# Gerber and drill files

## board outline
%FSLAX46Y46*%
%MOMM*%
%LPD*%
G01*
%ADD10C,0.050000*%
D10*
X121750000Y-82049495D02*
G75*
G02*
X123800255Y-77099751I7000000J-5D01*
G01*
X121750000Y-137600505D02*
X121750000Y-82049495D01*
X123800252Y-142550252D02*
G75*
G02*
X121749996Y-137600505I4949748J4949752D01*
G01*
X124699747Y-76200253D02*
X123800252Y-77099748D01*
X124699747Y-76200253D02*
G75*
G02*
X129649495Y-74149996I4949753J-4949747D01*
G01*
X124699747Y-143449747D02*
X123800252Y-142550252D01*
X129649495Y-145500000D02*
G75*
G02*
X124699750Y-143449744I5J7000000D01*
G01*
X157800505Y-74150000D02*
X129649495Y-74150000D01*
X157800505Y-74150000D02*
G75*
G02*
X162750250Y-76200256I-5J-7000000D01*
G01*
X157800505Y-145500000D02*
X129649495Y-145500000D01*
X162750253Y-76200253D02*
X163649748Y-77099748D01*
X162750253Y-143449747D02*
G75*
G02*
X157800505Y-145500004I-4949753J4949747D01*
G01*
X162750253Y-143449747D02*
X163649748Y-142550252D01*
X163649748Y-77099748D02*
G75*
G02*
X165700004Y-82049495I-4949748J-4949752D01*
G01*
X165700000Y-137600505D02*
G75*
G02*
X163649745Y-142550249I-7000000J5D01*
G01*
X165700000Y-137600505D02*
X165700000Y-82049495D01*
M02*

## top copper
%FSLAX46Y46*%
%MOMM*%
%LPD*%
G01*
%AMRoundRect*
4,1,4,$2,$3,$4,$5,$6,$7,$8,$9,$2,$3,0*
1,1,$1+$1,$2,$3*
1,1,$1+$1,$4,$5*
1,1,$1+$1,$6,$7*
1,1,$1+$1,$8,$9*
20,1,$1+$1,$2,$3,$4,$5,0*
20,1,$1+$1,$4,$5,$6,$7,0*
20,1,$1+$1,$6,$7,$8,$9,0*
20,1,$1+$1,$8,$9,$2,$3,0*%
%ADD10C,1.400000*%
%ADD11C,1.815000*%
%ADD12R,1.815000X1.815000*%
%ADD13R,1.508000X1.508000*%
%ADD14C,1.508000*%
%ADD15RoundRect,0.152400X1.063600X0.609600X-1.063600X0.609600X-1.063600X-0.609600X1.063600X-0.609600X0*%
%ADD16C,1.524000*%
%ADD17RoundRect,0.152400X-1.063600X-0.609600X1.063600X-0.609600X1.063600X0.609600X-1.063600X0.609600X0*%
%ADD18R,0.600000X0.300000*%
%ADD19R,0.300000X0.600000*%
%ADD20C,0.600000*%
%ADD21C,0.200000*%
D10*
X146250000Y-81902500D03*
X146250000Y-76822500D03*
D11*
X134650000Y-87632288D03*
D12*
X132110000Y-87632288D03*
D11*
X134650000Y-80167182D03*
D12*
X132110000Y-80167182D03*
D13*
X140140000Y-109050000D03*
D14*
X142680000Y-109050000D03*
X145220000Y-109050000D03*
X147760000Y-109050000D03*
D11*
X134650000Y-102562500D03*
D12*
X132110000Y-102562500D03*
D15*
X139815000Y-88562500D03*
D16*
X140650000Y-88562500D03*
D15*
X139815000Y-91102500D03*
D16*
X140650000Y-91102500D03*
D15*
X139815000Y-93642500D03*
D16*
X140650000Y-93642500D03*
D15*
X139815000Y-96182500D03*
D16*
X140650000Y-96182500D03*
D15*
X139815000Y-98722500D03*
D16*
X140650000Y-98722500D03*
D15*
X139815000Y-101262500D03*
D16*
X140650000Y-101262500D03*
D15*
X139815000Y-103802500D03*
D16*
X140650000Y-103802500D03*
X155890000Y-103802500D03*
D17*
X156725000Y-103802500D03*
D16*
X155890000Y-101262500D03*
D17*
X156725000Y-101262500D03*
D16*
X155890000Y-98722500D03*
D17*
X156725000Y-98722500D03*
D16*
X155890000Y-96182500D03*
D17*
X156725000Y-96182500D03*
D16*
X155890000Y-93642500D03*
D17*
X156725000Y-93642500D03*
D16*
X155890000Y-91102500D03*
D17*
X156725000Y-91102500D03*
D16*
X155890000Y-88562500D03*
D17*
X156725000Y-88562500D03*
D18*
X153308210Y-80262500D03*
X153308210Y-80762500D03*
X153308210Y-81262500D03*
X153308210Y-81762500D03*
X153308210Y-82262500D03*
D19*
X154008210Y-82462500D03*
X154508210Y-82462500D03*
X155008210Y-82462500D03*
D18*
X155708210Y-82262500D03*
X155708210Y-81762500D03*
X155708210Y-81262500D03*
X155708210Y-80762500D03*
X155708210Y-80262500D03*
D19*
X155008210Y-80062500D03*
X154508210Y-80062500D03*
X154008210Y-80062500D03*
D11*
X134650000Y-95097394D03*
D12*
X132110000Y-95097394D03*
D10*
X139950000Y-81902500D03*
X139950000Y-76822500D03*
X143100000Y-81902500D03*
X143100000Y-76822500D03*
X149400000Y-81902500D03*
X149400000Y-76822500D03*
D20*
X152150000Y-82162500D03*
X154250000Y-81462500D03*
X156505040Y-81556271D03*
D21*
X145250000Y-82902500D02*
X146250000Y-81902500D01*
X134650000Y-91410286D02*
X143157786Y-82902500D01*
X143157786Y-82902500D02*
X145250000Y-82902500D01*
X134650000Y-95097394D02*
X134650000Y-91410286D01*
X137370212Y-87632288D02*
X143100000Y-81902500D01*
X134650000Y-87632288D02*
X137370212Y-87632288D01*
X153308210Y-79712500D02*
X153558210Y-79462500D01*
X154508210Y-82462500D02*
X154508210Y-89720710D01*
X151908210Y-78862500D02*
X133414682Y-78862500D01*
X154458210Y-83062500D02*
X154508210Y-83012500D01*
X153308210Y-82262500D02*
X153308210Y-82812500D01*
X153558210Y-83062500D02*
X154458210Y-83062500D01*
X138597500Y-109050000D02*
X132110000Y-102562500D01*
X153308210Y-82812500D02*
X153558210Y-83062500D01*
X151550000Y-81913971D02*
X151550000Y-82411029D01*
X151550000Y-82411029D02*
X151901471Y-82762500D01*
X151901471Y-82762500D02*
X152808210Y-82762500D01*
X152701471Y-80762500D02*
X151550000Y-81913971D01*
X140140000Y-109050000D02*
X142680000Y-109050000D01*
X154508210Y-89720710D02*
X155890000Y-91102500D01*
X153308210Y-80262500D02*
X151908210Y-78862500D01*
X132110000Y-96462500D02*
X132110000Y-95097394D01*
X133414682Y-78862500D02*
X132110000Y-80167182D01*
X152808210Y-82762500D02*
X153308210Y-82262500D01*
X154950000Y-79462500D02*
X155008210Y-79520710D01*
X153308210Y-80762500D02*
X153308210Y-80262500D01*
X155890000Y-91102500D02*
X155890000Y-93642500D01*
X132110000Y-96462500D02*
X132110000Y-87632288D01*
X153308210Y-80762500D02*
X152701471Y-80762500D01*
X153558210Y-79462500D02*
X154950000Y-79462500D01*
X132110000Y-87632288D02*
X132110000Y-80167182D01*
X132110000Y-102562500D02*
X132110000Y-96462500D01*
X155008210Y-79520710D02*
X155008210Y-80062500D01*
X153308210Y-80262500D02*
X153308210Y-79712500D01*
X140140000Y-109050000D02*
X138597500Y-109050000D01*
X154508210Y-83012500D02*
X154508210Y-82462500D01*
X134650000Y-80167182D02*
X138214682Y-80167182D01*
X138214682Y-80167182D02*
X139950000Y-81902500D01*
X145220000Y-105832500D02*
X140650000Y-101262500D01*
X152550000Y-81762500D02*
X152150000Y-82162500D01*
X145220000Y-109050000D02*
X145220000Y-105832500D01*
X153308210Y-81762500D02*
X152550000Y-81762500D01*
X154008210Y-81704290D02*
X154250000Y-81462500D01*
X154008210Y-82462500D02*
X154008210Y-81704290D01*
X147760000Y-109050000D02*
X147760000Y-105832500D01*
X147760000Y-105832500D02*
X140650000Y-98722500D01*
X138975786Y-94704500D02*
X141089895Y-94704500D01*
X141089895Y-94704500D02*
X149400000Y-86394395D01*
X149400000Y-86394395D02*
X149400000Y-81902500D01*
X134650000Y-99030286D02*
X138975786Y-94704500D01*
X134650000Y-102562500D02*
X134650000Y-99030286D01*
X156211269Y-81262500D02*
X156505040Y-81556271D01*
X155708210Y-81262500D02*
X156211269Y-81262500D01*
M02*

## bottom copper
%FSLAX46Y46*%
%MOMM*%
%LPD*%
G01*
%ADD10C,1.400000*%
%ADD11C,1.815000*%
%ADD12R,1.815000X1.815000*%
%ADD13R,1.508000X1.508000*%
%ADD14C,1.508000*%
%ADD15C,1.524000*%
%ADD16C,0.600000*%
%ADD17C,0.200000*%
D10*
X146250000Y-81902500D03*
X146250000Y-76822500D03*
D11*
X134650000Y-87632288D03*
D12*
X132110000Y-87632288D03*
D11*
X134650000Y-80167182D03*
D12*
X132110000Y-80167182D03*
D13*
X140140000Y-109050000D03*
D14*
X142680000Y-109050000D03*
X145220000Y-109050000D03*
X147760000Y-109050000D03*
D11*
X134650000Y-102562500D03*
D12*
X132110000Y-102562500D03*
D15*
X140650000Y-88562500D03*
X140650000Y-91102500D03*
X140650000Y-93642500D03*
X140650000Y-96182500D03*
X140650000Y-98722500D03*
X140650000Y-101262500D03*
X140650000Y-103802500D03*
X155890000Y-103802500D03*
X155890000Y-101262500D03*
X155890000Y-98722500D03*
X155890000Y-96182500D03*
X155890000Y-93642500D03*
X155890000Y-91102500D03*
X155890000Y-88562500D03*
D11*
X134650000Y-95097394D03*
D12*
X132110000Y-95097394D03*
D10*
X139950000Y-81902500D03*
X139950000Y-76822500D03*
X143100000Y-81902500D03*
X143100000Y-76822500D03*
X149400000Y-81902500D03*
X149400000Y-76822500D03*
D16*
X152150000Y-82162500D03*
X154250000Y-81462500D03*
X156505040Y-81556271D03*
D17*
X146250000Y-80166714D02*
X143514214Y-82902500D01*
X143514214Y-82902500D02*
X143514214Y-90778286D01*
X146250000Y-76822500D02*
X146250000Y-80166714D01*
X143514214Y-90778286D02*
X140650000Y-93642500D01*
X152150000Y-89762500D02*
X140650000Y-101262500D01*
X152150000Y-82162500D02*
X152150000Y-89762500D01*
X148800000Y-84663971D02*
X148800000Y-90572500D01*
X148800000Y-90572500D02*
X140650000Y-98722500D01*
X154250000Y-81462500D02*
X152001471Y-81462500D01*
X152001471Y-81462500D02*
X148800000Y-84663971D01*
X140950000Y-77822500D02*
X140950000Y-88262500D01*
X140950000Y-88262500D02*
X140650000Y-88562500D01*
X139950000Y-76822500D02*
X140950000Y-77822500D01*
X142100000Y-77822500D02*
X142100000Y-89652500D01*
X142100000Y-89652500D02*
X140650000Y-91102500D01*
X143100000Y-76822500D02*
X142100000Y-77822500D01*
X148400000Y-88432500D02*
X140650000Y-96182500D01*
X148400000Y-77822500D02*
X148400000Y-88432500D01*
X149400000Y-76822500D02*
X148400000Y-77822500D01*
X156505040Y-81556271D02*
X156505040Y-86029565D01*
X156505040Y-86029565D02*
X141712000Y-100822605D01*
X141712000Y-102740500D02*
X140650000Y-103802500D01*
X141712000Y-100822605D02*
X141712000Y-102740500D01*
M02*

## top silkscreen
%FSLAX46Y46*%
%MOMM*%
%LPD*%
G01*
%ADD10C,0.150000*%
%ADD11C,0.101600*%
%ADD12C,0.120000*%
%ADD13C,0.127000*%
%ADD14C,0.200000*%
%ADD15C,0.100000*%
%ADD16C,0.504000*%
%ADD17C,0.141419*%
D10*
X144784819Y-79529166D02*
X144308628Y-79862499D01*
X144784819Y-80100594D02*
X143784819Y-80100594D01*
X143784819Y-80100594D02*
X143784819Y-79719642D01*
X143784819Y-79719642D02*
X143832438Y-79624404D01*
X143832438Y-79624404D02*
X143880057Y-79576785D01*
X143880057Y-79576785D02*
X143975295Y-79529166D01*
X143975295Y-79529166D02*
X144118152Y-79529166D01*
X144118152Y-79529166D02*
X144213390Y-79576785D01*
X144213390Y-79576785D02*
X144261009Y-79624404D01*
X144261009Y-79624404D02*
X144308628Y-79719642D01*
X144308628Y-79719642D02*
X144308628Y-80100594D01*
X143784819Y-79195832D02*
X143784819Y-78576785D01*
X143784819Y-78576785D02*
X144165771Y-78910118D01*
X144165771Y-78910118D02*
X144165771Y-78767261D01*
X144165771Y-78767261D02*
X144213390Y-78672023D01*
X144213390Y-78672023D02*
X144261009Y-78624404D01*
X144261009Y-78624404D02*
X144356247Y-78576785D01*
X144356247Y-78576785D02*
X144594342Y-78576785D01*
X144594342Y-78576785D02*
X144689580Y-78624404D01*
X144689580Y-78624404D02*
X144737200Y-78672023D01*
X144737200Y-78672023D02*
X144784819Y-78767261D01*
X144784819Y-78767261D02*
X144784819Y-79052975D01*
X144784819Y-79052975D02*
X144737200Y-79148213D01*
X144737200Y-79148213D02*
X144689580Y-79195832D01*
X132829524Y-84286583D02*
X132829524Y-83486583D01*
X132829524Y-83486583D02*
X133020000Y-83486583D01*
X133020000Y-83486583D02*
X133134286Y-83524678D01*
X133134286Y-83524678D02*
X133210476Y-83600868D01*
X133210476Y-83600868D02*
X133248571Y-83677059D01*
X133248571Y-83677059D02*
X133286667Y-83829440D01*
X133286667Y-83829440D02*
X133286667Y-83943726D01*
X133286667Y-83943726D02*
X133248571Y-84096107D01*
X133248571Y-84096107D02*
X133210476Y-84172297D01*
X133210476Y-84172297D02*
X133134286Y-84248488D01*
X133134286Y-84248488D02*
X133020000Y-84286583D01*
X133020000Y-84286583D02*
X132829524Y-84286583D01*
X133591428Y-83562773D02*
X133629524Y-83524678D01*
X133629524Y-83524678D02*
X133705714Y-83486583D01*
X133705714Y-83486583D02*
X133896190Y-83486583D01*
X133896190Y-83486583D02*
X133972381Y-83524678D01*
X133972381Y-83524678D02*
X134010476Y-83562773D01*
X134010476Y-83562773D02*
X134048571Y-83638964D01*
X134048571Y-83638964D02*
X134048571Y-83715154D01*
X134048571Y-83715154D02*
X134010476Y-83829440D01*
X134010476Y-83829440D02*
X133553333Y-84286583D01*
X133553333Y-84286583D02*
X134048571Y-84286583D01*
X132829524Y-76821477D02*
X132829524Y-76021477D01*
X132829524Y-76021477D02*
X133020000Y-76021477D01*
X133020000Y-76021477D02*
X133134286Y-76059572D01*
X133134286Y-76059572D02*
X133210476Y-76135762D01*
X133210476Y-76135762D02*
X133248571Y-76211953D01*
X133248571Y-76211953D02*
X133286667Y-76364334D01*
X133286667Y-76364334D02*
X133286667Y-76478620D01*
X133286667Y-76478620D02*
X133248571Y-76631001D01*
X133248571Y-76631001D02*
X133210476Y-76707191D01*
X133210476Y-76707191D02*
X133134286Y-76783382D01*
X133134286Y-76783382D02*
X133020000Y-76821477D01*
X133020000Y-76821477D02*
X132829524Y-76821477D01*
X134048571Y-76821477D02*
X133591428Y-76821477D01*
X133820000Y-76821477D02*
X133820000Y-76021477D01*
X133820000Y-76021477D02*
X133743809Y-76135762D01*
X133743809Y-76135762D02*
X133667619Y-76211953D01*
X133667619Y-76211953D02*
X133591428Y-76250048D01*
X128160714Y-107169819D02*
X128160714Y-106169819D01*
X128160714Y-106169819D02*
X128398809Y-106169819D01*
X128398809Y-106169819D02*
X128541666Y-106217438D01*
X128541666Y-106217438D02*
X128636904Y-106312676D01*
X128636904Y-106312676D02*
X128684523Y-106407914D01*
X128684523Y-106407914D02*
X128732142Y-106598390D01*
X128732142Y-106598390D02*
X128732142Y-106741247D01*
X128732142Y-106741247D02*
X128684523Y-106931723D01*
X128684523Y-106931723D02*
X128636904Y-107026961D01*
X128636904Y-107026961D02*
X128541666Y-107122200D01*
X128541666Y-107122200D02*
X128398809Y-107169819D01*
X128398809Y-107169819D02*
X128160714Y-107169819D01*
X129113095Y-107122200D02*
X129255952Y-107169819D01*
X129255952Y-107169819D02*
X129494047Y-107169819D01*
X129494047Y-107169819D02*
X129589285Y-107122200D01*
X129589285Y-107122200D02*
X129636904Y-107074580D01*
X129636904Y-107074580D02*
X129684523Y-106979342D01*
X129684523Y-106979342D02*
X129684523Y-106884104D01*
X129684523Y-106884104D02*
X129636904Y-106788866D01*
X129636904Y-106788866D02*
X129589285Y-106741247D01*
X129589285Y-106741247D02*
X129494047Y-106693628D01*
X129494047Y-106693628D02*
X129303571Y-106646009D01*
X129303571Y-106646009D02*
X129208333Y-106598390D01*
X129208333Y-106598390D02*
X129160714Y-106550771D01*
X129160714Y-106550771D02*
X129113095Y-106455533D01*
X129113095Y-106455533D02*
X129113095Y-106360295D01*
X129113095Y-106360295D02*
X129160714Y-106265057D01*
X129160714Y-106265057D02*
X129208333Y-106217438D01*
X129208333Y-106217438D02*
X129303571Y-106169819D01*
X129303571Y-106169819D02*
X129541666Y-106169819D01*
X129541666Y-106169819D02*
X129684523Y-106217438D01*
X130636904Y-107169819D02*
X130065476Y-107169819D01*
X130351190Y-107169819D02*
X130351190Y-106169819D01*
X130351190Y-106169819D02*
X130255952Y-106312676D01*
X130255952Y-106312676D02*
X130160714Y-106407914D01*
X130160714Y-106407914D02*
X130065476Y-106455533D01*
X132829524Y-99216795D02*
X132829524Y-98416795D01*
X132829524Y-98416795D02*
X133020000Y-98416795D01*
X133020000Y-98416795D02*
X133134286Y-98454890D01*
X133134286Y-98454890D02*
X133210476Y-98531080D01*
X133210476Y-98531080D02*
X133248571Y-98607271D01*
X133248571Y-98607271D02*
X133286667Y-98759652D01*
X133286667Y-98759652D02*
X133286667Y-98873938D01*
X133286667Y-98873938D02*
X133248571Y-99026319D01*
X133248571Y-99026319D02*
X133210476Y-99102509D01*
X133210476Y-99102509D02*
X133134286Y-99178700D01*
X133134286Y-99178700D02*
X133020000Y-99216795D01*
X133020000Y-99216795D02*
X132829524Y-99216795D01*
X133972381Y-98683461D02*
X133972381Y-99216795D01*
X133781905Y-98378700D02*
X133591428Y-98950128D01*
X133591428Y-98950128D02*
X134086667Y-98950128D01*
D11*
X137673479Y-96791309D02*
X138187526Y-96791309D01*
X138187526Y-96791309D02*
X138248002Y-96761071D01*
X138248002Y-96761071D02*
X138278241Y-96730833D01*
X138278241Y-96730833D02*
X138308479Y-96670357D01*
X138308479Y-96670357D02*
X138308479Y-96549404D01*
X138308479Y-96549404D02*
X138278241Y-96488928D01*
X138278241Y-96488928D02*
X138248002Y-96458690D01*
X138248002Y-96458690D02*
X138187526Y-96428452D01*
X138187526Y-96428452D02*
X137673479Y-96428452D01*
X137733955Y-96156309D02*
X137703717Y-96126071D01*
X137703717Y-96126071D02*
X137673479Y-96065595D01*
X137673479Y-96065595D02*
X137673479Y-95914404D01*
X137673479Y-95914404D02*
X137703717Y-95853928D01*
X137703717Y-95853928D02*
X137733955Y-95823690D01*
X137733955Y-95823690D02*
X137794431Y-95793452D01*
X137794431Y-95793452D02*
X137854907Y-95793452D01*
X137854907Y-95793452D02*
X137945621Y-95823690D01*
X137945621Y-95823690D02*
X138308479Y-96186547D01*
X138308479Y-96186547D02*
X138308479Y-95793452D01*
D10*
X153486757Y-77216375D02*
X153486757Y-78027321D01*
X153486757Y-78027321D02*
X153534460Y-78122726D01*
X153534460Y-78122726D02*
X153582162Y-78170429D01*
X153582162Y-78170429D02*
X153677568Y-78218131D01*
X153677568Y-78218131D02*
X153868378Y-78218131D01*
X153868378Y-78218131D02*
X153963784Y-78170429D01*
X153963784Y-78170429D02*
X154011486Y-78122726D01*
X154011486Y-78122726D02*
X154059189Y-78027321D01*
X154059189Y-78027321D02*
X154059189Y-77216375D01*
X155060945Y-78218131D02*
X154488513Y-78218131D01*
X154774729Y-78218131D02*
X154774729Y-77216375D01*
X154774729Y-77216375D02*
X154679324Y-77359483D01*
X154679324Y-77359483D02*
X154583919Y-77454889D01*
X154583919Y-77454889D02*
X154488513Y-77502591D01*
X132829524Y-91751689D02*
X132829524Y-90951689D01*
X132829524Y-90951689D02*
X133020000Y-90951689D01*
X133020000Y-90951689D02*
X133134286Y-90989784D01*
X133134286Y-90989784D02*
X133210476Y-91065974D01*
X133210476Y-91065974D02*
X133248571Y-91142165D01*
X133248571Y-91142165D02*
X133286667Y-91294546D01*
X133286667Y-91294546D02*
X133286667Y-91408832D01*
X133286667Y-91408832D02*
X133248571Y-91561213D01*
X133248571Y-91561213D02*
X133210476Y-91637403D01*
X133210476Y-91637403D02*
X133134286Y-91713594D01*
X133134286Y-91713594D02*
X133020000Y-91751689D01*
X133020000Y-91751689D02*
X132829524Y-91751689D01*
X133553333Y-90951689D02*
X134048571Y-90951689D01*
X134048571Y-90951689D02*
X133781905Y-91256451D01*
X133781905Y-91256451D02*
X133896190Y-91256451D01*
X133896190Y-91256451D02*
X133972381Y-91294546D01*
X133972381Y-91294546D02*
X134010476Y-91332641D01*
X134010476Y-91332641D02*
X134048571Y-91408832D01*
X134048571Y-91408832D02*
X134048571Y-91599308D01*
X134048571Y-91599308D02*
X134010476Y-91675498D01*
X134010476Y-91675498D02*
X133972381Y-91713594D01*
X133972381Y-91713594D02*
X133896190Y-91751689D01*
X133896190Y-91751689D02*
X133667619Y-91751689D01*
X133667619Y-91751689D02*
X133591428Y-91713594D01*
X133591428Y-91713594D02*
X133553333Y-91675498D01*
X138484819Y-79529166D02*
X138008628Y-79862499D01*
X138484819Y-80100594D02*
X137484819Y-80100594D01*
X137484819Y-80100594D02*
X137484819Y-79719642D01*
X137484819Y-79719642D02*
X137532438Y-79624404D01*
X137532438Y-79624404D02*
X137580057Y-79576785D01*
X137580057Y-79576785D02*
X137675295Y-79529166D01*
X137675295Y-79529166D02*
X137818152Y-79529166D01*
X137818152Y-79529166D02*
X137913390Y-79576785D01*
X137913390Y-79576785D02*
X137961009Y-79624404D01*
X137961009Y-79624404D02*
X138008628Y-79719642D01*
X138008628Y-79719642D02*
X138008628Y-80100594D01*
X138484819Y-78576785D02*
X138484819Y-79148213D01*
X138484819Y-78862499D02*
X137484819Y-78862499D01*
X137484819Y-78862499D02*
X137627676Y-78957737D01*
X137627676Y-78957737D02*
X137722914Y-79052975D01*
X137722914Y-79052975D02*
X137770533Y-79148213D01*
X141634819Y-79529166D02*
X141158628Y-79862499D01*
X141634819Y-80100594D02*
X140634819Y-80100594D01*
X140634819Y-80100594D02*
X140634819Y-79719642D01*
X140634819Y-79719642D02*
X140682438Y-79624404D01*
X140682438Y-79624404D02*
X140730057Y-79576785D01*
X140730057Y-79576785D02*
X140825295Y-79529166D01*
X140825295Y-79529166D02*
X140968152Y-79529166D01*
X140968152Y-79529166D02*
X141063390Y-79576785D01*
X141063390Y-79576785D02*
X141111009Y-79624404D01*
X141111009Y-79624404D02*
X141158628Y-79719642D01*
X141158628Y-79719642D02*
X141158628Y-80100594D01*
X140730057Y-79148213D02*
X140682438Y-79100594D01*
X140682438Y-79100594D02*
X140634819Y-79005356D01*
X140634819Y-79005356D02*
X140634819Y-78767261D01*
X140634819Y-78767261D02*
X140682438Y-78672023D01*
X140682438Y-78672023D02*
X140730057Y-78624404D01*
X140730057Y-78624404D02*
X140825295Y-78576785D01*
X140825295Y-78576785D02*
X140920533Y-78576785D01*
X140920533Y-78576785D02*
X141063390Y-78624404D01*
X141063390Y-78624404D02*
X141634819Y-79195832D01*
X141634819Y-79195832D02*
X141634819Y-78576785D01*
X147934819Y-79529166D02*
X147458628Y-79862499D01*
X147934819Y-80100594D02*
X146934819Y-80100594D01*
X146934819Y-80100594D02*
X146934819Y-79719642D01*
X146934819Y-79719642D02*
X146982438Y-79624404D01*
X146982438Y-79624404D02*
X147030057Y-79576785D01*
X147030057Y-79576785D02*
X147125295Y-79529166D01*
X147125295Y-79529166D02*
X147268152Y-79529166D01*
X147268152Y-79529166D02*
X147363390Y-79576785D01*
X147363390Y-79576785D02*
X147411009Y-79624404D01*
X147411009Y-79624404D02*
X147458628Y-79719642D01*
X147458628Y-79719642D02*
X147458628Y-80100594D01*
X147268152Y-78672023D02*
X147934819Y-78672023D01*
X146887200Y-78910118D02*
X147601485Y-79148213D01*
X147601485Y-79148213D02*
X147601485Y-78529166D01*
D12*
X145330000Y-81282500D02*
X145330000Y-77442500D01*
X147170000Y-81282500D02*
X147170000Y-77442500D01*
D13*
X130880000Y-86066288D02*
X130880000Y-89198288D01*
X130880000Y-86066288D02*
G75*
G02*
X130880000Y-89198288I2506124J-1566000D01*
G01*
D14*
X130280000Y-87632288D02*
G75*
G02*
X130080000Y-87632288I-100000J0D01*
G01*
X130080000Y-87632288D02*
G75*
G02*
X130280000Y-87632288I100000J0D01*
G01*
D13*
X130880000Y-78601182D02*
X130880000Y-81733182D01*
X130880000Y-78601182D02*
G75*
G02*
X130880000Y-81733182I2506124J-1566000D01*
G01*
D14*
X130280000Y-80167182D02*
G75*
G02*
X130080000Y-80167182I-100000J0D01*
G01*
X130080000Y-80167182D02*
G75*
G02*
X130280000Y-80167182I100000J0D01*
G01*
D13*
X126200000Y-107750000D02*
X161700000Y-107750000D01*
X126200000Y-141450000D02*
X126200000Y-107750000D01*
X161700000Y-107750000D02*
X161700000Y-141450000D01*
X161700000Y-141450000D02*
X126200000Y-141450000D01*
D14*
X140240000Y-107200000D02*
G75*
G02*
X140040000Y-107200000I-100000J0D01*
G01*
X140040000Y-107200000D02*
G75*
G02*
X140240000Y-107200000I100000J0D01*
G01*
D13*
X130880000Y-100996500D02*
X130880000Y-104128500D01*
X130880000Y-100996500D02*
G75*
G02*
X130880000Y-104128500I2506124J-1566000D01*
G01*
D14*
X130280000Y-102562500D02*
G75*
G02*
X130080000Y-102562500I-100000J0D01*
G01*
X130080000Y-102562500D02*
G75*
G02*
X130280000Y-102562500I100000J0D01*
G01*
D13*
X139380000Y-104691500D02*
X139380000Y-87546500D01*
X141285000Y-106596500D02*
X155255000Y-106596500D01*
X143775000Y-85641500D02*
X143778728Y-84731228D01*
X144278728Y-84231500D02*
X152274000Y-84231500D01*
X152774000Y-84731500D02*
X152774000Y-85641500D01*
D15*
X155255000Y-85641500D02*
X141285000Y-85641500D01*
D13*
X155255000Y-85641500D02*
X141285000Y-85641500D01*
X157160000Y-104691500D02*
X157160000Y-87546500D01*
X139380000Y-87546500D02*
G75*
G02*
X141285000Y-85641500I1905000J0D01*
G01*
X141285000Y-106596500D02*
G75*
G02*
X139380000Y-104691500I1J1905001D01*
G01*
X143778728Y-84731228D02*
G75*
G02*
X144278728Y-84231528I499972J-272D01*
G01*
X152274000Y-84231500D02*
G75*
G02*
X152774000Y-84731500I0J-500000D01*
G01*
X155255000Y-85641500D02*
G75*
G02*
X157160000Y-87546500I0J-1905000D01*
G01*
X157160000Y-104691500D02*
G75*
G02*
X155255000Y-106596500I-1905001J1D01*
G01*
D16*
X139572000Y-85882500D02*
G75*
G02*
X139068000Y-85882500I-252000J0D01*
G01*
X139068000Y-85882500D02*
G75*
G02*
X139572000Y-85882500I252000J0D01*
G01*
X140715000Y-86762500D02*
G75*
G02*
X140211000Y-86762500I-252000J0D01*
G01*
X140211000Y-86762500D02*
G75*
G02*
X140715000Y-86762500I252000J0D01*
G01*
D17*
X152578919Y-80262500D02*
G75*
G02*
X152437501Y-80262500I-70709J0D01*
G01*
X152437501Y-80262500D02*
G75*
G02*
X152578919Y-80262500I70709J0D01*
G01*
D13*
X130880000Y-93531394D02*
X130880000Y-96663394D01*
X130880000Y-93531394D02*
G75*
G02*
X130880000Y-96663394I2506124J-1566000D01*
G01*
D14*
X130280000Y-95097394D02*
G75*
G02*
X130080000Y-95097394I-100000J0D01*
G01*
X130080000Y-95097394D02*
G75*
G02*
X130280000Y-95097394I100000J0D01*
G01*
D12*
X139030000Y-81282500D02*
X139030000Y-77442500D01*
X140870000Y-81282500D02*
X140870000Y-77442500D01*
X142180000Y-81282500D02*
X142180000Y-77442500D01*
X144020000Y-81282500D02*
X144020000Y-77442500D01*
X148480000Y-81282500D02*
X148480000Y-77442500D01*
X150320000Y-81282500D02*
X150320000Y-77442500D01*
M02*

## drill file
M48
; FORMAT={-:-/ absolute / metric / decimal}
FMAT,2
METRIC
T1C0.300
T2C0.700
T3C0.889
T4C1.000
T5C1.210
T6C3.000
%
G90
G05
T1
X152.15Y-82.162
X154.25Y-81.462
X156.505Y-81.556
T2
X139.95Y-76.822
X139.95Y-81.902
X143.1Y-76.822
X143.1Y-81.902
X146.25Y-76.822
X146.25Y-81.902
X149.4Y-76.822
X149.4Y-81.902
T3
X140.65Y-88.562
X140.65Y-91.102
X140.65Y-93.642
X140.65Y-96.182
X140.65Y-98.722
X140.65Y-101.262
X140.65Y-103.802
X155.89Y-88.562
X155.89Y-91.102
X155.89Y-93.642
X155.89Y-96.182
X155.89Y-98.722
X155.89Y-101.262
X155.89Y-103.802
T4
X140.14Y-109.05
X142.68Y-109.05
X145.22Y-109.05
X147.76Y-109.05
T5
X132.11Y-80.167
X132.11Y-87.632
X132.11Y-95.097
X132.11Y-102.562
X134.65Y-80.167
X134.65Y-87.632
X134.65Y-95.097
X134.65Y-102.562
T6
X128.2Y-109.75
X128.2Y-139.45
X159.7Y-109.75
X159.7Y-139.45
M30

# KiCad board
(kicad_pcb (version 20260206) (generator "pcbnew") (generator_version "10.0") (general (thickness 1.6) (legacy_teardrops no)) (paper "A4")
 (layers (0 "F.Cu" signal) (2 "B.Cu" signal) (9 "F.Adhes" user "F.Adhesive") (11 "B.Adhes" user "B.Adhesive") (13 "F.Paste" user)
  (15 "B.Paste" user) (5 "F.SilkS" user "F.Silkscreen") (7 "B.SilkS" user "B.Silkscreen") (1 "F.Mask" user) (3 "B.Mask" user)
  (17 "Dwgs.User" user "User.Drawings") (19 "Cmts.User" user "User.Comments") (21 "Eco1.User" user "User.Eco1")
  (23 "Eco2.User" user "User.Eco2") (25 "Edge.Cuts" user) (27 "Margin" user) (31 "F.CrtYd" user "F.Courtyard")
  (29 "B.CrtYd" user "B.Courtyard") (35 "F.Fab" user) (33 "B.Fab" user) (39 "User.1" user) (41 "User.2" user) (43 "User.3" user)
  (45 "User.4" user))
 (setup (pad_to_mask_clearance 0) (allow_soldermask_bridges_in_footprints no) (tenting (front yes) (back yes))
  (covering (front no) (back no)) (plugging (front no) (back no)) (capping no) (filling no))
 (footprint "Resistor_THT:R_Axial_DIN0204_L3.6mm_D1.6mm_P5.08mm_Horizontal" (layer "F.Cu") (at 146.25 81.9025 90)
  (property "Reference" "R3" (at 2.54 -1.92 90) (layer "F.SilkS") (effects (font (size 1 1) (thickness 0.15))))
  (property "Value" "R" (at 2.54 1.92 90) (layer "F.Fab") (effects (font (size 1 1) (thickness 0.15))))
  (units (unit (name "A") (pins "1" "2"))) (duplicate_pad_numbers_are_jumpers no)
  (fp_line (start 0.62 -0.92) (end 4.46 -0.92) (stroke (width 0.12) (type solid)) (layer "F.SilkS"))
  (fp_line (start 0.62 0.92) (end 4.46 0.92) (stroke (width 0.12) (type solid)) (layer "F.SilkS"))
  (pad "1" thru_hole circle (at 0 0 90) (size 1.4 1.4) (drill 0.7) (layers "*.Cu" "*.Mask") (remove_unused_layers no) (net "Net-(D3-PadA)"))
  (pad "2" thru_hole circle (at 5.08 0 90) (size 1.4 1.4) (drill 0.7) (layers "*.Cu" "*.Mask") (remove_unused_layers no) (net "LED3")))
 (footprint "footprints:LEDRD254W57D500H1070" (layer "F.Cu") (at 133.38 87.632288)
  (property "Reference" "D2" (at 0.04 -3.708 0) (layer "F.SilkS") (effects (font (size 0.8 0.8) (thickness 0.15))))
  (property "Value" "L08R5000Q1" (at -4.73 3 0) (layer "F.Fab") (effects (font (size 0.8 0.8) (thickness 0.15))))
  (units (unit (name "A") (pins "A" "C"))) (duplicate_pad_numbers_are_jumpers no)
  (fp_line (start -2.5 -1.566) (end -2.5 1.566) (stroke (width 0.127) (type solid)) (layer "F.SilkS"))
  (fp_arc (start -2.5 -1.566) (mid 2.961291 0) (end -2.5 1.566) (stroke (width 0.127) (type solid)) (layer "F.SilkS"))
  (fp_circle (center -3.2 0) (end -3.1 0) (stroke (width 0.2) (type solid)) (fill no) (layer "F.SilkS"))
  (pad "A" thru_hole circle (at 1.27 0) (size 1.815 1.815) (drill 1.21) (layers "*.Cu" "*.Mask") (remove_unused_layers no)
   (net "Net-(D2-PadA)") (solder_mask_margin 0.102))
  (pad "C" thru_hole rect (at -1.27 0) (size 1.815 1.815) (drill 1.21) (layers "*.Cu" "*.Mask") (remove_unused_layers no) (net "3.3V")
   (solder_mask_margin 0.102)))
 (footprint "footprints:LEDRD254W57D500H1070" (layer "F.Cu") (at 133.38 80.167182)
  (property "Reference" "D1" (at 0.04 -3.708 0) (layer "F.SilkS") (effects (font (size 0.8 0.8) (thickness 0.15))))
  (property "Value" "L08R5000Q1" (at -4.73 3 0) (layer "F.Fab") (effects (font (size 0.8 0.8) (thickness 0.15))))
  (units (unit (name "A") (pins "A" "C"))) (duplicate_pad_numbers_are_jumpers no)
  (fp_line (start -2.5 -1.566) (end -2.5 1.566) (stroke (width 0.127) (type solid)) (layer "F.SilkS"))
  (fp_arc (start -2.5 -1.566) (mid 2.961291 0) (end -2.5 1.566) (stroke (width 0.127) (type solid)) (layer "F.SilkS"))
  (fp_circle (center -3.2 0) (end -3.1 0) (stroke (width 0.2) (type solid)) (fill no) (layer "F.SilkS"))
  (pad "A" thru_hole circle (at 1.27 0) (size 1.815 1.815) (drill 1.21) (layers "*.Cu" "*.Mask") (remove_unused_layers no)
   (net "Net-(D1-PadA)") (solder_mask_margin 0.102))
  (pad "C" thru_hole rect (at -1.27 0) (size 1.815 1.815) (drill 1.21) (layers "*.Cu" "*.Mask") (remove_unused_layers no) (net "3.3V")
   (solder_mask_margin 0.102)))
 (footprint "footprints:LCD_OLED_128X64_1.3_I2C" (layer "F.Cu") (at 143.95 124.6)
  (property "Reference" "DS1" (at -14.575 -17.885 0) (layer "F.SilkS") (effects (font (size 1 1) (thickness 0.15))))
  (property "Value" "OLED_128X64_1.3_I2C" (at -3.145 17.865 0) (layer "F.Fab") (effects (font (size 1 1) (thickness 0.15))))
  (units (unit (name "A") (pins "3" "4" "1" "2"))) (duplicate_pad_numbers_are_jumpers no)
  (fp_line (start -17.75 -16.85) (end 17.75 -16.85) (stroke (width 0.127) (type solid)) (layer "F.SilkS"))
  (fp_line (start -17.75 16.85) (end -17.75 -16.85) (stroke (width 0.127) (type solid)) (layer "F.SilkS"))
  (fp_line (start 17.75 -16.85) (end 17.75 16.85) (stroke (width 0.127) (type solid)) (layer "F.SilkS"))
  (fp_line (start 17.75 16.85) (end -17.75 16.85) (stroke (width 0.127) (type solid)) (layer "F.SilkS"))
  (fp_circle (center -3.81 -17.4) (end -3.71 -17.4) (stroke (width 0.2) (type solid)) (fill no) (layer "F.SilkS"))
  (pad "" np_thru_hole circle (at -15.75 -14.85) (size 3 3) (drill 3) (layers "*.Cu" "*.Mask"))
  (pad "" np_thru_hole circle (at -15.75 14.85) (size 3 3) (drill 3) (layers "*.Cu" "*.Mask"))
  (pad "" np_thru_hole circle (at 15.75 -14.85) (size 3 3) (drill 3) (layers "*.Cu" "*.Mask"))
  (pad "" np_thru_hole circle (at 15.75 14.85) (size 3 3) (drill 3) (layers "*.Cu" "*.Mask"))
  (pad "1" thru_hole rect (at -3.81 -15.55) (size 1.508 1.508) (drill 1) (layers "*.Cu" "*.Mask") (remove_unused_layers no) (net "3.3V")
   (solder_mask_margin 0.102))
  (pad "2" thru_hole circle (at -1.27 -15.55) (size 1.508 1.508) (drill 1) (layers "*.Cu" "*.Mask") (remove_unused_layers no) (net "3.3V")
   (solder_mask_margin 0.102))
  (pad "3" thru_hole circle (at 1.27 -15.55) (size 1.508 1.508) (drill 1) (layers "*.Cu" "*.Mask") (remove_unused_layers no) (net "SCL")
   (solder_mask_margin 0.102))
  (pad "4" thru_hole circle (at 3.81 -15.55) (size 1.508 1.508) (drill 1) (layers "*.Cu" "*.Mask") (remove_unused_layers no) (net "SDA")
   (solder_mask_margin 0.102)))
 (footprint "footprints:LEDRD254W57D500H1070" (layer "F.Cu") (at 133.38 102.5625)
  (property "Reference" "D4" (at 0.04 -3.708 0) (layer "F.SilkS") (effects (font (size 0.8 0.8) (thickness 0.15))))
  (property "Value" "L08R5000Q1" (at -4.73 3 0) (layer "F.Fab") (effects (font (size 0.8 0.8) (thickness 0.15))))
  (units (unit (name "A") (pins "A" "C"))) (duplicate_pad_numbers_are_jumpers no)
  (fp_line (start -2.5 -1.566) (end -2.5 1.566) (stroke (width 0.127) (type solid)) (layer "F.SilkS"))
  (fp_arc (start -2.5 -1.566) (mid 2.961291 0) (end -2.5 1.566) (stroke (width 0.127) (type solid)) (layer "F.SilkS"))
  (fp_circle (center -3.2 0) (end -3.1 0) (stroke (width 0.2) (type solid)) (fill no) (layer "F.SilkS"))
  (pad "A" thru_hole circle (at 1.27 0) (size 1.815 1.815) (drill 1.21) (layers "*.Cu" "*.Mask") (remove_unused_layers no)
   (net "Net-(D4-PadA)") (solder_mask_margin 0.102))
  (pad "C" thru_hole rect (at -1.27 0) (size 1.815 1.815) (drill 1.21) (layers "*.Cu" "*.Mask") (remove_unused_layers no) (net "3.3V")
   (solder_mask_margin 0.102)))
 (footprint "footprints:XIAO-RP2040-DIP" (layer "F.Cu") (at 148.27 96.1825 90)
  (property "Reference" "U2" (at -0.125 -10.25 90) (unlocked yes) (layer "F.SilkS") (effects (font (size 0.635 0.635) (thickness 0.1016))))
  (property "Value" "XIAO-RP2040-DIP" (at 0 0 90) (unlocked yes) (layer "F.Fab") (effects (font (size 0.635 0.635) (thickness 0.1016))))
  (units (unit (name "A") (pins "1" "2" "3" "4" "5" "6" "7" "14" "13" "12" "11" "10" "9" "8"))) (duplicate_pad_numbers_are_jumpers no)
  (fp_line (start -8.509 -8.89) (end 8.636 -8.89) (stroke (width 0.127) (type solid)) (layer "F.SilkS"))
  (fp_line (start -10.414 -6.985) (end -10.414 6.985) (stroke (width 0.127) (type solid)) (layer "F.SilkS"))
  (fp_line (start 10.541 -4.495) (end 11.451272 -4.491272) (stroke (width 0.127) (type solid)) (layer "F.SilkS"))
  (fp_line (start 11.951 -3.991272) (end 11.951 4.004) (stroke (width 0.127) (type solid)) (layer "F.SilkS"))
  (fp_line (start 11.451 4.504) (end 10.541 4.504) (stroke (width 0.127) (type solid)) (layer "F.SilkS"))
  (fp_line (start 10.541 6.985) (end 10.541 -6.985) (stroke (width 0.1) (type solid)) (layer "F.SilkS"))
  (fp_line (start 10.541 6.985) (end 10.541 -6.985) (stroke (width 0.127) (type solid)) (layer "F.SilkS"))
  (fp_line (start -8.509 8.89) (end 8.636 8.89) (stroke (width 0.127) (type solid)) (layer "F.SilkS"))
  (fp_arc (start 8.636 -8.89) (mid 9.983038 -8.332038) (end 10.541 -6.985) (stroke (width 0.127) (type solid)) (layer "F.SilkS"))
  (fp_arc (start -10.414 -6.985) (mid -9.856038 -8.332038) (end -8.509 -8.89) (stroke (width 0.127) (type solid)) (layer "F.SilkS"))
  (fp_arc (start 11.451272 -4.491272) (mid 11.804644 -4.344724) (end 11.951 -3.991272) (stroke (width 0.127) (type default))
   (layer "F.SilkS"))
  (fp_arc (start 11.951 4.004) (mid 11.804553 4.357553) (end 11.451 4.504) (stroke (width 0.127) (type default)) (layer "F.SilkS"))
  (fp_arc (start 10.541 6.985) (mid 9.983038 8.332038) (end 8.636 8.89) (stroke (width 0.127) (type solid)) (layer "F.SilkS"))
  (fp_arc (start -8.509 8.89) (mid -9.856038 8.332038) (end -10.414 6.985) (stroke (width 0.127) (type solid)) (layer "F.SilkS"))
  (fp_circle (center 10.3 -8.95) (end 10.554 -8.95) (stroke (width 0.5) (type solid)) (fill yes) (layer "F.SilkS"))
  (fp_circle (center 9.42 -7.807) (end 9.674 -7.807) (stroke (width 0.5) (type solid)) (fill yes) (layer "F.SilkS"))
  (pad "1" smd roundrect (at 7.62 -8.455 180) (size 2.432 1.524) (layers "F.Cu" "F.Mask") (roundrect_rratio 0.1) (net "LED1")
   (thermal_bridge_angle 45))
  (pad "1" thru_hole circle (at 7.62 -7.62 180) (size 1.524 1.524) (drill 0.889) (layers "*.Cu" "*.Mask") (remove_unused_layers no)
   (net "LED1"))
  (pad "2" smd roundrect (at 5.08 -8.455 180) (size 2.432 1.524) (layers "F.Cu" "F.Mask") (roundrect_rratio 0.1) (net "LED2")
   (thermal_bridge_angle 45))
  (pad "2" thru_hole circle (at 5.08 -7.62 180) (size 1.524 1.524) (drill 0.889) (layers "*.Cu" "*.Mask") (remove_unused_layers no)
   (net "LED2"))
  (pad "3" smd roundrect (at 2.54 -8.455 180) (size 2.432 1.524) (layers "F.Cu" "F.Mask") (roundrect_rratio 0.1) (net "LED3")
   (thermal_bridge_angle 45))
  (pad "3" thru_hole circle (at 2.54 -7.62 180) (size 1.524 1.524) (drill 0.889) (layers "*.Cu" "*.Mask") (remove_unused_layers no)
   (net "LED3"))
  (pad "4" smd roundrect (at 0 -8.455 180) (size 2.432 1.524) (layers "F.Cu" "F.Mask") (roundrect_rratio 0.1) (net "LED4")
   (thermal_bridge_angle 45))
  (pad "4" thru_hole circle (at 0 -7.62 180) (size 1.524 1.524) (drill 0.889) (layers "*.Cu" "*.Mask") (remove_unused_layers no)
   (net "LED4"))
  (pad "5" smd roundrect (at -2.54 -8.455 180) (size 2.432 1.524) (layers "F.Cu" "F.Mask") (roundrect_rratio 0.1) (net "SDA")
   (thermal_bridge_angle 45))
  (pad "5" thru_hole circle (at -2.54 -7.62 180) (size 1.524 1.524) (drill 0.889) (layers "*.Cu" "*.Mask") (remove_unused_layers no)
   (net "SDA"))
  (pad "6" smd roundrect (at -5.08 -8.455 180) (size 2.432 1.524) (layers "F.Cu" "F.Mask") (roundrect_rratio 0.1) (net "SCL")
   (thermal_bridge_angle 45))
  (pad "6" thru_hole circle (at -5.08 -7.62 180) (size 1.524 1.524) (drill 0.889) (layers "*.Cu" "*.Mask") (remove_unused_layers no)
   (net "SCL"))
  (pad "7" smd roundrect (at -7.62 -8.455 180) (size 2.432 1.524) (layers "F.Cu" "F.Mask") (roundrect_rratio 0.1) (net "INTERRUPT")
   (thermal_bridge_angle 45))
  (pad "7" thru_hole circle (at -7.62 -7.62 180) (size 1.524 1.524) (drill 0.889) (layers "*.Cu" "*.Mask") (remove_unused_layers no)
   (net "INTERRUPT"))
  (pad "8" thru_hole circle (at -7.62 7.62) (size 1.524 1.524) (drill 0.889) (layers "*.Cu" "*.Mask") (remove_unused_layers no)
   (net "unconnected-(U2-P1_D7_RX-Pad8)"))
  (pad "8" smd roundrect (at -7.62 8.455) (size 2.432 1.524) (layers "F.Cu" "F.Mask") (roundrect_rratio 0.1)
   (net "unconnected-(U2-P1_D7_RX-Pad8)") (thermal_bridge_angle 45))
  (pad "9" thru_hole circle (at -5.08 7.62) (size 1.524 1.524) (drill 0.889) (layers "*.Cu" "*.Mask") (remove_unused_layers no)
   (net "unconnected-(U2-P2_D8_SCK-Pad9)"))
  (pad "9" smd roundrect (at -5.08 8.455) (size 2.432 1.524) (layers "F.Cu" "F.Mask") (roundrect_rratio 0.1)
   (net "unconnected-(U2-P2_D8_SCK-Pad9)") (thermal_bridge_angle 45))
  (pad "10" thru_hole circle (at -2.54 7.62) (size 1.524 1.524) (drill 0.889) (layers "*.Cu" "*.Mask") (remove_unused_layers no)
   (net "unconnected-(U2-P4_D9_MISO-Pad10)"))
  (pad "10" smd roundrect (at -2.54 8.455) (size 2.432 1.524) (layers "F.Cu" "F.Mask") (roundrect_rratio 0.1)
   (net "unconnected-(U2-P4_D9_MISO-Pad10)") (thermal_bridge_angle 45))
  (pad "11" thru_hole circle (at 0 7.62) (size 1.524 1.524) (drill 0.889) (layers "*.Cu" "*.Mask") (remove_unused_layers no)
   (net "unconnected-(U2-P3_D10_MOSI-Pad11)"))
  (pad "11" smd roundrect (at 0 8.455) (size 2.432 1.524) (layers "F.Cu" "F.Mask") (roundrect_rratio 0.1)
   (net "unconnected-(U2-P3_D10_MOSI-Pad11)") (thermal_bridge_angle 45))
  (pad "12" thru_hole circle (at 2.54 7.62) (size 1.524 1.524) (drill 0.889) (layers "*.Cu" "*.Mask") (remove_unused_layers no) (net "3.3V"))
  (pad "12" smd roundrect (at 2.54 8.455) (size 2.432 1.524) (layers "F.Cu" "F.Mask") (roundrect_rratio 0.1) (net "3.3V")
   (thermal_bridge_angle 45))
  (pad "13" thru_hole circle (at 5.08 7.62) (size 1.524 1.524) (drill 0.889) (layers "*.Cu" "*.Mask") (remove_unused_layers no) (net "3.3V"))
  (pad "13" smd roundrect (at 5.08 8.455) (size 2.432 1.524) (layers "F.Cu" "F.Mask") (roundrect_rratio 0.1) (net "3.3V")
   (thermal_bridge_angle 45))
  (pad "14" thru_hole circle (at 7.62 7.62) (size 1.524 1.524) (drill 0.889) (layers "*.Cu" "*.Mask") (remove_unused_layers no)
   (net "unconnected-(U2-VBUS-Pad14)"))
  (pad "14" smd roundrect (at 7.62 8.455) (size 2.432 1.524) (layers "F.Cu" "F.Mask") (roundrect_rratio 0.1)
   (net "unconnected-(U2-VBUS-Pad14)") (thermal_bridge_angle 45)))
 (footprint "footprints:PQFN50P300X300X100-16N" (layer "F.Cu") (at 154.50821 81.2625)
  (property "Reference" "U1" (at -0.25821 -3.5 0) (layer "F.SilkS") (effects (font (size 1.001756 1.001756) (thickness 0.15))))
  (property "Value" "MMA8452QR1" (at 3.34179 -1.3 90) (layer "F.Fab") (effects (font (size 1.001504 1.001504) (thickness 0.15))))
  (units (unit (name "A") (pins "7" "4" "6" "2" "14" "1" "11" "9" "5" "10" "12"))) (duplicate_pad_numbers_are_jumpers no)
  (fp_circle (center -2 -1) (end -1.858581 -1) (stroke (width 0) (type solid)) (fill yes) (layer "F.SilkS"))
  (pad "1" smd rect (at -1.2 -1) (size 0.6 0.3) (layers "F.Cu" "F.Mask" "F.Paste") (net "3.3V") (solder_mask_margin 0.102))
  (pad "2" smd rect (at -1.2 -0.5) (size 0.6 0.3) (layers "F.Cu" "F.Mask" "F.Paste") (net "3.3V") (solder_mask_margin 0.102))
  (pad "3" smd rect (at -1.2 0) (size 0.6 0.3) (layers "F.Cu" "F.Mask" "F.Paste") (solder_mask_margin 0.102))
  (pad "4" smd rect (at -1.2 0.5) (size 0.6 0.3) (layers "F.Cu" "F.Mask" "F.Paste") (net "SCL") (solder_mask_margin 0.102))
  (pad "5" smd rect (at -1.2 1) (size 0.6 0.3) (layers "F.Cu" "F.Mask" "F.Paste") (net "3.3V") (solder_mask_margin 0.102))
  (pad "6" smd rect (at -0.5 1.2) (size 0.3 0.6) (layers "F.Cu" "F.Mask" "F.Paste") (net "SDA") (solder_mask_margin 0.102))
  (pad "7" smd rect (at 0 1.2) (size 0.3 0.6) (layers "F.Cu" "F.Mask" "F.Paste") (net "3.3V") (solder_mask_margin 0.102))
  (pad "8" smd rect (at 0.5 1.2) (size 0.3 0.6) (layers "F.Cu" "F.Mask" "F.Paste") (solder_mask_margin 0.102))
  (pad "9" smd rect (at 1.2 1) (size 0.6 0.3) (layers "F.Cu" "F.Mask" "F.Paste") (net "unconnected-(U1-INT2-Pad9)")
   (solder_mask_margin 0.102))
  (pad "10" smd rect (at 1.2 0.5) (size 0.6 0.3) (layers "F.Cu" "F.Mask" "F.Paste") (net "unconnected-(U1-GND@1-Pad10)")
   (solder_mask_margin 0.102))
  (pad "11" smd rect (at 1.2 0) (size 0.6 0.3) (layers "F.Cu" "F.Mask" "F.Paste") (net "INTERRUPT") (solder_mask_margin 0.102))
  (pad "12" smd rect (at 1.2 -0.5) (size 0.6 0.3) (layers "F.Cu" "F.Mask" "F.Paste") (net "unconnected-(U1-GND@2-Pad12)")
   (solder_mask_margin 0.102))
  (pad "13" smd rect (at 1.2 -1) (size 0.6 0.3) (layers "F.Cu" "F.Mask" "F.Paste") (solder_mask_margin 0.102))
  (pad "14" smd rect (at 0.5 -1.2) (size 0.3 0.6) (layers "F.Cu" "F.Mask" "F.Paste") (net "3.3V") (solder_mask_margin 0.102))
  (pad "15" smd rect (at 0 -1.2) (size 0.3 0.6) (layers "F.Cu" "F.Mask" "F.Paste") (solder_mask_margin 0.102))
  (pad "16" smd rect (at -0.5 -1.2) (size 0.3 0.6) (layers "F.Cu" "F.Mask" "F.Paste") (solder_mask_margin 0.102)))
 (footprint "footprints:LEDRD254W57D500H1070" (layer "F.Cu") (at 133.38 95.097394)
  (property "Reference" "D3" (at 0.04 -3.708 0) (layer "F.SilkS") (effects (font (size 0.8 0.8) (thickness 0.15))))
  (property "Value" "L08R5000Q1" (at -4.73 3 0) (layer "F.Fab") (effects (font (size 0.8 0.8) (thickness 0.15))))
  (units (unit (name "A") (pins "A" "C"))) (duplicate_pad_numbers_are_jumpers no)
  (fp_line (start -2.5 -1.566) (end -2.5 1.566) (stroke (width 0.127) (type solid)) (layer "F.SilkS"))
  (fp_arc (start -2.5 -1.566) (mid 2.961291 0) (end -2.5 1.566) (stroke (width 0.127) (type solid)) (layer "F.SilkS"))
  (fp_circle (center -3.2 0) (end -3.1 0) (stroke (width 0.2) (type solid)) (fill no) (layer "F.SilkS"))
  (pad "A" thru_hole circle (at 1.27 0) (size 1.815 1.815) (drill 1.21) (layers "*.Cu" "*.Mask") (remove_unused_layers no)
   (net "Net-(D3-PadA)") (solder_mask_margin 0.102))
  (pad "C" thru_hole rect (at -1.27 0) (size 1.815 1.815) (drill 1.21) (layers "*.Cu" "*.Mask") (remove_unused_layers no) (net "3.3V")
   (solder_mask_margin 0.102)))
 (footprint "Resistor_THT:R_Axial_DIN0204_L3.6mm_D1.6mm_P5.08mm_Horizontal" (layer "F.Cu") (at 139.95 81.9025 90)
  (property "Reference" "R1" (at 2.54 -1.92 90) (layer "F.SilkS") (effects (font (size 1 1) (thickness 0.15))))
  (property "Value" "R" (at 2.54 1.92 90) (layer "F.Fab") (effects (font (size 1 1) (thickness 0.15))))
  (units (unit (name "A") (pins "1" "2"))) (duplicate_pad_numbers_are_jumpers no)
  (fp_line (start 0.62 -0.92) (end 4.46 -0.92) (stroke (width 0.12) (type solid)) (layer "F.SilkS"))
  (fp_line (start 0.62 0.92) (end 4.46 0.92) (stroke (width 0.12) (type solid)) (layer "F.SilkS"))
  (pad "1" thru_hole circle (at 0 0 90) (size 1.4 1.4) (drill 0.7) (layers "*.Cu" "*.Mask") (remove_unused_layers no) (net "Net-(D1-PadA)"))
  (pad "2" thru_hole circle (at 5.08 0 90) (size 1.4 1.4) (drill 0.7) (layers "*.Cu" "*.Mask") (remove_unused_layers no) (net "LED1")))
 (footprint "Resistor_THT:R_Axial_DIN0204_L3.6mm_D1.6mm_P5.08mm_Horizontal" (layer "F.Cu") (at 143.1 81.9025 90)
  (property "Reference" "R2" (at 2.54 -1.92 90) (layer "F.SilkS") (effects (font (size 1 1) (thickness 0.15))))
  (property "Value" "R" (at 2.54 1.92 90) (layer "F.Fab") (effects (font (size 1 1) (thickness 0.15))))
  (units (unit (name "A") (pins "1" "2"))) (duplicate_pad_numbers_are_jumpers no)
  (fp_line (start 0.62 -0.92) (end 4.46 -0.92) (stroke (width 0.12) (type solid)) (layer "F.SilkS"))
  (fp_line (start 0.62 0.92) (end 4.46 0.92) (stroke (width 0.12) (type solid)) (layer "F.SilkS"))
  (pad "1" thru_hole circle (at 0 0 90) (size 1.4 1.4) (drill 0.7) (layers "*.Cu" "*.Mask") (remove_unused_layers no) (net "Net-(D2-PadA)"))
  (pad "2" thru_hole circle (at 5.08 0 90) (size 1.4 1.4) (drill 0.7) (layers "*.Cu" "*.Mask") (remove_unused_layers no) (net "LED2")))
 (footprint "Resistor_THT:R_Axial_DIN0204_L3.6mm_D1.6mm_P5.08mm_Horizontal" (layer "F.Cu") (at 149.4 81.9025 90)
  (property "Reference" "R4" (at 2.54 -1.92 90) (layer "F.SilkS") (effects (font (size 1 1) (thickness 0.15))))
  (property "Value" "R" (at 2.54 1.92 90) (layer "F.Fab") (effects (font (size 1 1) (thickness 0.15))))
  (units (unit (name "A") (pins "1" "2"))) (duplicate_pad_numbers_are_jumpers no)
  (fp_line (start 0.62 -0.92) (end 4.46 -0.92) (stroke (width 0.12) (type solid)) (layer "F.SilkS"))
  (fp_line (start 0.62 0.92) (end 4.46 0.92) (stroke (width 0.12) (type solid)) (layer "F.SilkS"))
  (pad "1" thru_hole circle (at 0 0 90) (size 1.4 1.4) (drill 0.7) (layers "*.Cu" "*.Mask") (remove_unused_layers no) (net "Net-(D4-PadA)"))
  (pad "2" thru_hole circle (at 5.08 0 90) (size 1.4 1.4) (drill 0.7) (layers "*.Cu" "*.Mask") (remove_unused_layers no) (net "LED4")))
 (gr_arc (start 121.75 82.049495) (mid 122.282845 79.370712) (end 123.800252 77.099748) (stroke (width 0.05) (type default))
  (layer "Edge.Cuts"))
 (gr_line (start 121.75 137.600505) (end 121.75 82.049495) (stroke (width 0.05) (type default)) (layer "Edge.Cuts"))
 (gr_arc (start 123.800252 142.550252) (mid 122.282843 140.279289) (end 121.75 137.600505) (stroke (width 0.05) (type default))
  (layer "Edge.Cuts"))
 (gr_line (start 124.699747 76.200253) (end 123.800252 77.099748) (stroke (width 0.05) (type default)) (layer "Edge.Cuts"))
 (gr_arc (start 124.699747 76.200253) (mid 126.97071 74.682842) (end 129.649495 74.15) (stroke (width 0.05) (type default))
  (layer "Edge.Cuts"))
 (gr_line (start 124.699747 143.449747) (end 123.800252 142.550252) (stroke (width 0.05) (type default)) (layer "Edge.Cuts"))
 (gr_arc (start 129.649495 145.5) (mid 126.970711 144.967157) (end 124.699747 143.449747) (stroke (width 0.05) (type default))
  (layer "Edge.Cuts"))
 (gr_line (start 157.800505 74.15) (end 129.649495 74.15) (stroke (width 0.05) (type default)) (layer "Edge.Cuts"))
 (gr_arc (start 157.800505 74.15) (mid 160.479289 74.682843) (end 162.750253 76.200253) (stroke (width 0.05) (type default))
  (layer "Edge.Cuts"))
 (gr_line (start 157.800505 145.5) (end 129.649495 145.5) (stroke (width 0.05) (type default)) (layer "Edge.Cuts"))
 (gr_line (start 162.750253 76.200253) (end 163.649748 77.099748) (stroke (width 0.05) (type default)) (layer "Edge.Cuts"))
 (gr_arc (start 162.750253 143.449747) (mid 160.47929 144.967158) (end 157.800505 145.5) (stroke (width 0.05) (type default))
  (layer "Edge.Cuts"))
 (gr_line (start 162.750253 143.449747) (end 163.649748 142.550252) (stroke (width 0.05) (type default)) (layer "Edge.Cuts"))
 (gr_arc (start 163.649748 77.099748) (mid 165.167159 79.370711) (end 165.7 82.049495) (stroke (width 0.05) (type default))
  (layer "Edge.Cuts"))
 (gr_arc (start 165.7 137.600505) (mid 165.167157 140.279289) (end 163.649748 142.550252) (stroke (width 0.05) (type default))
  (layer "Edge.Cuts"))
 (gr_line (start 165.7 137.600505) (end 165.7 82.049495) (stroke (width 0.05) (type default)) (layer "Edge.Cuts"))
 (segment (start 145.25 82.9025) (end 146.25 81.9025) (width 0.2) (layer "F.Cu") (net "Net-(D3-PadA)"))
 (segment (start 134.65 91.410286) (end 143.157786 82.9025) (width 0.2) (layer "F.Cu") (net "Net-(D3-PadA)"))
 (segment (start 143.157786 82.9025) (end 145.25 82.9025) (width 0.2) (layer "F.Cu") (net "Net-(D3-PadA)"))
 (segment (start 134.65 95.097394) (end 134.65 91.410286) (width 0.2) (layer "F.Cu") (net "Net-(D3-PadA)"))
 (segment (start 146.25 80.166714) (end 143.514214 82.9025) (width 0.2) (layer "B.Cu") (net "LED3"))
 (segment (start 143.514214 82.9025) (end 143.514214 90.778286) (width 0.2) (layer "B.Cu") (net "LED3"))
 (segment (start 146.25 76.8225) (end 146.25 80.166714) (width 0.2) (layer "B.Cu") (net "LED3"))
 (segment (start 143.514214 90.778286) (end 140.65 93.6425) (width 0.2) (layer "B.Cu") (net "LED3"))
 (segment (start 137.370212 87.632288) (end 143.1 81.9025) (width 0.2) (layer "F.Cu") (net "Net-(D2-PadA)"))
 (segment (start 134.65 87.632288) (end 137.370212 87.632288) (width 0.2) (layer "F.Cu") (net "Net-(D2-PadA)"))
 (segment (start 153.30821 79.7125) (end 153.55821 79.4625) (width 0.2) (layer "F.Cu") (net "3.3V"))
 (segment (start 154.50821 82.4625) (end 154.50821 89.72071) (width 0.2) (layer "F.Cu") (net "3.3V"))
 (segment (start 151.90821 78.8625) (end 133.414682 78.8625) (width 0.2) (layer "F.Cu") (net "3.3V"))
 (segment (start 154.45821 83.0625) (end 154.50821 83.0125) (width 0.2) (layer "F.Cu") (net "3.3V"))
 (segment (start 153.30821 82.2625) (end 153.30821 82.8125) (width 0.2) (layer "F.Cu") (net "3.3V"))
 (segment (start 153.55821 83.0625) (end 154.45821 83.0625) (width 0.2) (layer "F.Cu") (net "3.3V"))
 (segment (start 138.5975 109.05) (end 132.11 102.5625) (width 0.2) (layer "F.Cu") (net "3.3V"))
 (segment (start 153.30821 82.8125) (end 153.55821 83.0625) (width 0.2) (layer "F.Cu") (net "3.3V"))
 (segment (start 151.55 81.913971) (end 151.55 82.411029) (width 0.2) (layer "F.Cu") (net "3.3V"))
 (segment (start 151.55 82.411029) (end 151.901471 82.7625) (width 0.2) (layer "F.Cu") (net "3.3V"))
 (segment (start 151.901471 82.7625) (end 152.80821 82.7625) (width 0.2) (layer "F.Cu") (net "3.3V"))
 (segment (start 152.701471 80.7625) (end 151.55 81.913971) (width 0.2) (layer "F.Cu") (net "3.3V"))
 (segment (start 140.14 109.05) (end 142.68 109.05) (width 0.2) (layer "F.Cu") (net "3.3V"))
 (segment (start 154.50821 89.72071) (end 155.89 91.1025) (width 0.2) (layer "F.Cu") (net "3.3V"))
 (segment (start 153.30821 80.2625) (end 151.90821 78.8625) (width 0.2) (layer "F.Cu") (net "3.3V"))
 (segment (start 132.11 96.4625) (end 132.11 95.097394) (width 0.2) (layer "F.Cu") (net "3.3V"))
 (segment (start 133.414682 78.8625) (end 132.11 80.167182) (width 0.2) (layer "F.Cu") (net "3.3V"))
 (segment (start 152.80821 82.7625) (end 153.30821 82.2625) (width 0.2) (layer "F.Cu") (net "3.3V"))
 (segment (start 154.95 79.4625) (end 155.00821 79.52071) (width 0.2) (layer "F.Cu") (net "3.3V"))
 (segment (start 153.30821 80.7625) (end 153.30821 80.2625) (width 0.2) (layer "F.Cu") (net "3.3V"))
 (segment (start 155.89 91.1025) (end 155.89 93.6425) (width 0.2) (layer "F.Cu") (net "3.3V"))
 (segment (start 132.11 96.4625) (end 132.11 87.632288) (width 0.2) (layer "F.Cu") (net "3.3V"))
 (segment (start 153.30821 80.7625) (end 152.701471 80.7625) (width 0.2) (layer "F.Cu") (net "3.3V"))
 (segment (start 153.55821 79.4625) (end 154.95 79.4625) (width 0.2) (layer "F.Cu") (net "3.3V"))
 (segment (start 132.11 87.632288) (end 132.11 80.167182) (width 0.2) (layer "F.Cu") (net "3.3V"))
 (segment (start 132.11 102.5625) (end 132.11 96.4625) (width 0.2) (layer "F.Cu") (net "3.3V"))
 (segment (start 155.00821 79.52071) (end 155.00821 80.0625) (width 0.2) (layer "F.Cu") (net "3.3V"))
 (segment (start 153.30821 80.2625) (end 153.30821 79.7125) (width 0.2) (layer "F.Cu") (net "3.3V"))
 (segment (start 140.14 109.05) (end 138.5975 109.05) (width 0.2) (layer "F.Cu") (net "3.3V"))
 (segment (start 154.50821 83.0125) (end 154.50821 82.4625) (width 0.2) (layer "F.Cu") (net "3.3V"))
 (segment (start 134.65 80.167182) (end 138.214682 80.167182) (width 0.2) (layer "F.Cu") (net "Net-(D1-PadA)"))
 (segment (start 138.214682 80.167182) (end 139.95 81.9025) (width 0.2) (layer "F.Cu") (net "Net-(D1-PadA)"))
 (segment (start 145.22 105.8325) (end 140.65 101.2625) (width 0.2) (layer "F.Cu") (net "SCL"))
 (segment (start 152.55 81.7625) (end 152.15 82.1625) (width 0.2) (layer "F.Cu") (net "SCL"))
 (segment (start 145.22 109.05) (end 145.22 105.8325) (width 0.2) (layer "F.Cu") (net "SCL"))
 (segment (start 153.30821 81.7625) (end 152.55 81.7625) (width 0.2) (layer "F.Cu") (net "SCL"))
 (via (at 152.15 82.1625) (size 0.6) (drill 0.3) (layers "F.Cu" "B.Cu") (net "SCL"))
 (segment (start 152.15 89.7625) (end 140.65 101.2625) (width 0.2) (layer "B.Cu") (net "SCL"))
 (segment (start 152.15 82.1625) (end 152.15 89.7625) (width 0.2) (layer "B.Cu") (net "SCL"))
 (segment (start 154.00821 81.70429) (end 154.25 81.4625) (width 0.2) (layer "F.Cu") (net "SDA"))
 (segment (start 154.00821 82.4625) (end 154.00821 81.70429) (width 0.2) (layer "F.Cu") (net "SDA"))
 (segment (start 147.76 109.05) (end 147.76 105.8325) (width 0.2) (layer "F.Cu") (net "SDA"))
 (segment (start 147.76 105.8325) (end 140.65 98.7225) (width 0.2) (layer "F.Cu") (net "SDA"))
 (via (at 154.25 81.4625) (size 0.6) (drill 0.3) (layers "F.Cu" "B.Cu") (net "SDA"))
 (segment (start 148.8 84.663971) (end 148.8 90.5725) (width 0.2) (layer "B.Cu") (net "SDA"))
 (segment (start 148.8 90.5725) (end 140.65 98.7225) (width 0.2) (layer "B.Cu") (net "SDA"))
 (segment (start 154.25 81.4625) (end 152.001471 81.4625) (width 0.2) (layer "B.Cu") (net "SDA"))
 (segment (start 152.001471 81.4625) (end 148.8 84.663971) (width 0.2) (layer "B.Cu") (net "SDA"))
 (segment (start 138.975786 94.7045) (end 141.089895 94.7045) (width 0.2) (layer "F.Cu") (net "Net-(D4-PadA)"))
 (segment (start 141.089895 94.7045) (end 149.4 86.394395) (width 0.2) (layer "F.Cu") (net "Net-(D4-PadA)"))
 (segment (start 149.4 86.394395) (end 149.4 81.9025) (width 0.2) (layer "F.Cu") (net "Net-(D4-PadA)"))
 (segment (start 134.65 99.030286) (end 138.975786 94.7045) (width 0.2) (layer "F.Cu") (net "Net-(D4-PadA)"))
 (segment (start 134.65 102.5625) (end 134.65 99.030286) (width 0.2) (layer "F.Cu") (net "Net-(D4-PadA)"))
 (segment (start 140.95 77.8225) (end 140.95 88.2625) (width 0.2) (layer "B.Cu") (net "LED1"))
 (segment (start 140.95 88.2625) (end 140.65 88.5625) (width 0.2) (layer "B.Cu") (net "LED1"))
 (segment (start 139.95 76.8225) (end 140.95 77.8225) (width 0.2) (layer "B.Cu") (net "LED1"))
 (segment (start 142.1 77.8225) (end 142.1 89.6525) (width 0.2) (layer "B.Cu") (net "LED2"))
 (segment (start 142.1 89.6525) (end 140.65 91.1025) (width 0.2) (layer "B.Cu") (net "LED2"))
 (segment (start 143.1 76.8225) (end 142.1 77.8225) (width 0.2) (layer "B.Cu") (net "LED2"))
 (segment (start 148.4 88.4325) (end 140.65 96.1825) (width 0.2) (layer "B.Cu") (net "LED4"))
 (segment (start 148.4 77.8225) (end 148.4 88.4325) (width 0.2) (layer "B.Cu") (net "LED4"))
 (segment (start 149.4 76.8225) (end 148.4 77.8225) (width 0.2) (layer "B.Cu") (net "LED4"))
 (segment (start 156.211269 81.2625) (end 156.50504 81.556271) (width 0.2) (layer "F.Cu") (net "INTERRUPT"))
 (segment (start 155.70821 81.2625) (end 156.211269 81.2625) (width 0.2) (layer "F.Cu") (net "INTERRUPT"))
 (via (at 156.50504 81.556271) (size 0.6) (drill 0.3) (layers "F.Cu" "B.Cu") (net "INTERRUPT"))
 (segment (start 156.50504 81.556271) (end 156.50504 86.029565) (width 0.2) (layer "B.Cu") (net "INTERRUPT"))
 (segment (start 156.50504 86.029565) (end 141.712 100.822605) (width 0.2) (layer "B.Cu") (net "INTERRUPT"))
 (segment (start 141.712 102.7405) (end 140.65 103.8025) (width 0.2) (layer "B.Cu") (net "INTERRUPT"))
 (segment (start 141.712 100.822605) (end 141.712 102.7405) (width 0.2) (layer "B.Cu") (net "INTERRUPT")))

